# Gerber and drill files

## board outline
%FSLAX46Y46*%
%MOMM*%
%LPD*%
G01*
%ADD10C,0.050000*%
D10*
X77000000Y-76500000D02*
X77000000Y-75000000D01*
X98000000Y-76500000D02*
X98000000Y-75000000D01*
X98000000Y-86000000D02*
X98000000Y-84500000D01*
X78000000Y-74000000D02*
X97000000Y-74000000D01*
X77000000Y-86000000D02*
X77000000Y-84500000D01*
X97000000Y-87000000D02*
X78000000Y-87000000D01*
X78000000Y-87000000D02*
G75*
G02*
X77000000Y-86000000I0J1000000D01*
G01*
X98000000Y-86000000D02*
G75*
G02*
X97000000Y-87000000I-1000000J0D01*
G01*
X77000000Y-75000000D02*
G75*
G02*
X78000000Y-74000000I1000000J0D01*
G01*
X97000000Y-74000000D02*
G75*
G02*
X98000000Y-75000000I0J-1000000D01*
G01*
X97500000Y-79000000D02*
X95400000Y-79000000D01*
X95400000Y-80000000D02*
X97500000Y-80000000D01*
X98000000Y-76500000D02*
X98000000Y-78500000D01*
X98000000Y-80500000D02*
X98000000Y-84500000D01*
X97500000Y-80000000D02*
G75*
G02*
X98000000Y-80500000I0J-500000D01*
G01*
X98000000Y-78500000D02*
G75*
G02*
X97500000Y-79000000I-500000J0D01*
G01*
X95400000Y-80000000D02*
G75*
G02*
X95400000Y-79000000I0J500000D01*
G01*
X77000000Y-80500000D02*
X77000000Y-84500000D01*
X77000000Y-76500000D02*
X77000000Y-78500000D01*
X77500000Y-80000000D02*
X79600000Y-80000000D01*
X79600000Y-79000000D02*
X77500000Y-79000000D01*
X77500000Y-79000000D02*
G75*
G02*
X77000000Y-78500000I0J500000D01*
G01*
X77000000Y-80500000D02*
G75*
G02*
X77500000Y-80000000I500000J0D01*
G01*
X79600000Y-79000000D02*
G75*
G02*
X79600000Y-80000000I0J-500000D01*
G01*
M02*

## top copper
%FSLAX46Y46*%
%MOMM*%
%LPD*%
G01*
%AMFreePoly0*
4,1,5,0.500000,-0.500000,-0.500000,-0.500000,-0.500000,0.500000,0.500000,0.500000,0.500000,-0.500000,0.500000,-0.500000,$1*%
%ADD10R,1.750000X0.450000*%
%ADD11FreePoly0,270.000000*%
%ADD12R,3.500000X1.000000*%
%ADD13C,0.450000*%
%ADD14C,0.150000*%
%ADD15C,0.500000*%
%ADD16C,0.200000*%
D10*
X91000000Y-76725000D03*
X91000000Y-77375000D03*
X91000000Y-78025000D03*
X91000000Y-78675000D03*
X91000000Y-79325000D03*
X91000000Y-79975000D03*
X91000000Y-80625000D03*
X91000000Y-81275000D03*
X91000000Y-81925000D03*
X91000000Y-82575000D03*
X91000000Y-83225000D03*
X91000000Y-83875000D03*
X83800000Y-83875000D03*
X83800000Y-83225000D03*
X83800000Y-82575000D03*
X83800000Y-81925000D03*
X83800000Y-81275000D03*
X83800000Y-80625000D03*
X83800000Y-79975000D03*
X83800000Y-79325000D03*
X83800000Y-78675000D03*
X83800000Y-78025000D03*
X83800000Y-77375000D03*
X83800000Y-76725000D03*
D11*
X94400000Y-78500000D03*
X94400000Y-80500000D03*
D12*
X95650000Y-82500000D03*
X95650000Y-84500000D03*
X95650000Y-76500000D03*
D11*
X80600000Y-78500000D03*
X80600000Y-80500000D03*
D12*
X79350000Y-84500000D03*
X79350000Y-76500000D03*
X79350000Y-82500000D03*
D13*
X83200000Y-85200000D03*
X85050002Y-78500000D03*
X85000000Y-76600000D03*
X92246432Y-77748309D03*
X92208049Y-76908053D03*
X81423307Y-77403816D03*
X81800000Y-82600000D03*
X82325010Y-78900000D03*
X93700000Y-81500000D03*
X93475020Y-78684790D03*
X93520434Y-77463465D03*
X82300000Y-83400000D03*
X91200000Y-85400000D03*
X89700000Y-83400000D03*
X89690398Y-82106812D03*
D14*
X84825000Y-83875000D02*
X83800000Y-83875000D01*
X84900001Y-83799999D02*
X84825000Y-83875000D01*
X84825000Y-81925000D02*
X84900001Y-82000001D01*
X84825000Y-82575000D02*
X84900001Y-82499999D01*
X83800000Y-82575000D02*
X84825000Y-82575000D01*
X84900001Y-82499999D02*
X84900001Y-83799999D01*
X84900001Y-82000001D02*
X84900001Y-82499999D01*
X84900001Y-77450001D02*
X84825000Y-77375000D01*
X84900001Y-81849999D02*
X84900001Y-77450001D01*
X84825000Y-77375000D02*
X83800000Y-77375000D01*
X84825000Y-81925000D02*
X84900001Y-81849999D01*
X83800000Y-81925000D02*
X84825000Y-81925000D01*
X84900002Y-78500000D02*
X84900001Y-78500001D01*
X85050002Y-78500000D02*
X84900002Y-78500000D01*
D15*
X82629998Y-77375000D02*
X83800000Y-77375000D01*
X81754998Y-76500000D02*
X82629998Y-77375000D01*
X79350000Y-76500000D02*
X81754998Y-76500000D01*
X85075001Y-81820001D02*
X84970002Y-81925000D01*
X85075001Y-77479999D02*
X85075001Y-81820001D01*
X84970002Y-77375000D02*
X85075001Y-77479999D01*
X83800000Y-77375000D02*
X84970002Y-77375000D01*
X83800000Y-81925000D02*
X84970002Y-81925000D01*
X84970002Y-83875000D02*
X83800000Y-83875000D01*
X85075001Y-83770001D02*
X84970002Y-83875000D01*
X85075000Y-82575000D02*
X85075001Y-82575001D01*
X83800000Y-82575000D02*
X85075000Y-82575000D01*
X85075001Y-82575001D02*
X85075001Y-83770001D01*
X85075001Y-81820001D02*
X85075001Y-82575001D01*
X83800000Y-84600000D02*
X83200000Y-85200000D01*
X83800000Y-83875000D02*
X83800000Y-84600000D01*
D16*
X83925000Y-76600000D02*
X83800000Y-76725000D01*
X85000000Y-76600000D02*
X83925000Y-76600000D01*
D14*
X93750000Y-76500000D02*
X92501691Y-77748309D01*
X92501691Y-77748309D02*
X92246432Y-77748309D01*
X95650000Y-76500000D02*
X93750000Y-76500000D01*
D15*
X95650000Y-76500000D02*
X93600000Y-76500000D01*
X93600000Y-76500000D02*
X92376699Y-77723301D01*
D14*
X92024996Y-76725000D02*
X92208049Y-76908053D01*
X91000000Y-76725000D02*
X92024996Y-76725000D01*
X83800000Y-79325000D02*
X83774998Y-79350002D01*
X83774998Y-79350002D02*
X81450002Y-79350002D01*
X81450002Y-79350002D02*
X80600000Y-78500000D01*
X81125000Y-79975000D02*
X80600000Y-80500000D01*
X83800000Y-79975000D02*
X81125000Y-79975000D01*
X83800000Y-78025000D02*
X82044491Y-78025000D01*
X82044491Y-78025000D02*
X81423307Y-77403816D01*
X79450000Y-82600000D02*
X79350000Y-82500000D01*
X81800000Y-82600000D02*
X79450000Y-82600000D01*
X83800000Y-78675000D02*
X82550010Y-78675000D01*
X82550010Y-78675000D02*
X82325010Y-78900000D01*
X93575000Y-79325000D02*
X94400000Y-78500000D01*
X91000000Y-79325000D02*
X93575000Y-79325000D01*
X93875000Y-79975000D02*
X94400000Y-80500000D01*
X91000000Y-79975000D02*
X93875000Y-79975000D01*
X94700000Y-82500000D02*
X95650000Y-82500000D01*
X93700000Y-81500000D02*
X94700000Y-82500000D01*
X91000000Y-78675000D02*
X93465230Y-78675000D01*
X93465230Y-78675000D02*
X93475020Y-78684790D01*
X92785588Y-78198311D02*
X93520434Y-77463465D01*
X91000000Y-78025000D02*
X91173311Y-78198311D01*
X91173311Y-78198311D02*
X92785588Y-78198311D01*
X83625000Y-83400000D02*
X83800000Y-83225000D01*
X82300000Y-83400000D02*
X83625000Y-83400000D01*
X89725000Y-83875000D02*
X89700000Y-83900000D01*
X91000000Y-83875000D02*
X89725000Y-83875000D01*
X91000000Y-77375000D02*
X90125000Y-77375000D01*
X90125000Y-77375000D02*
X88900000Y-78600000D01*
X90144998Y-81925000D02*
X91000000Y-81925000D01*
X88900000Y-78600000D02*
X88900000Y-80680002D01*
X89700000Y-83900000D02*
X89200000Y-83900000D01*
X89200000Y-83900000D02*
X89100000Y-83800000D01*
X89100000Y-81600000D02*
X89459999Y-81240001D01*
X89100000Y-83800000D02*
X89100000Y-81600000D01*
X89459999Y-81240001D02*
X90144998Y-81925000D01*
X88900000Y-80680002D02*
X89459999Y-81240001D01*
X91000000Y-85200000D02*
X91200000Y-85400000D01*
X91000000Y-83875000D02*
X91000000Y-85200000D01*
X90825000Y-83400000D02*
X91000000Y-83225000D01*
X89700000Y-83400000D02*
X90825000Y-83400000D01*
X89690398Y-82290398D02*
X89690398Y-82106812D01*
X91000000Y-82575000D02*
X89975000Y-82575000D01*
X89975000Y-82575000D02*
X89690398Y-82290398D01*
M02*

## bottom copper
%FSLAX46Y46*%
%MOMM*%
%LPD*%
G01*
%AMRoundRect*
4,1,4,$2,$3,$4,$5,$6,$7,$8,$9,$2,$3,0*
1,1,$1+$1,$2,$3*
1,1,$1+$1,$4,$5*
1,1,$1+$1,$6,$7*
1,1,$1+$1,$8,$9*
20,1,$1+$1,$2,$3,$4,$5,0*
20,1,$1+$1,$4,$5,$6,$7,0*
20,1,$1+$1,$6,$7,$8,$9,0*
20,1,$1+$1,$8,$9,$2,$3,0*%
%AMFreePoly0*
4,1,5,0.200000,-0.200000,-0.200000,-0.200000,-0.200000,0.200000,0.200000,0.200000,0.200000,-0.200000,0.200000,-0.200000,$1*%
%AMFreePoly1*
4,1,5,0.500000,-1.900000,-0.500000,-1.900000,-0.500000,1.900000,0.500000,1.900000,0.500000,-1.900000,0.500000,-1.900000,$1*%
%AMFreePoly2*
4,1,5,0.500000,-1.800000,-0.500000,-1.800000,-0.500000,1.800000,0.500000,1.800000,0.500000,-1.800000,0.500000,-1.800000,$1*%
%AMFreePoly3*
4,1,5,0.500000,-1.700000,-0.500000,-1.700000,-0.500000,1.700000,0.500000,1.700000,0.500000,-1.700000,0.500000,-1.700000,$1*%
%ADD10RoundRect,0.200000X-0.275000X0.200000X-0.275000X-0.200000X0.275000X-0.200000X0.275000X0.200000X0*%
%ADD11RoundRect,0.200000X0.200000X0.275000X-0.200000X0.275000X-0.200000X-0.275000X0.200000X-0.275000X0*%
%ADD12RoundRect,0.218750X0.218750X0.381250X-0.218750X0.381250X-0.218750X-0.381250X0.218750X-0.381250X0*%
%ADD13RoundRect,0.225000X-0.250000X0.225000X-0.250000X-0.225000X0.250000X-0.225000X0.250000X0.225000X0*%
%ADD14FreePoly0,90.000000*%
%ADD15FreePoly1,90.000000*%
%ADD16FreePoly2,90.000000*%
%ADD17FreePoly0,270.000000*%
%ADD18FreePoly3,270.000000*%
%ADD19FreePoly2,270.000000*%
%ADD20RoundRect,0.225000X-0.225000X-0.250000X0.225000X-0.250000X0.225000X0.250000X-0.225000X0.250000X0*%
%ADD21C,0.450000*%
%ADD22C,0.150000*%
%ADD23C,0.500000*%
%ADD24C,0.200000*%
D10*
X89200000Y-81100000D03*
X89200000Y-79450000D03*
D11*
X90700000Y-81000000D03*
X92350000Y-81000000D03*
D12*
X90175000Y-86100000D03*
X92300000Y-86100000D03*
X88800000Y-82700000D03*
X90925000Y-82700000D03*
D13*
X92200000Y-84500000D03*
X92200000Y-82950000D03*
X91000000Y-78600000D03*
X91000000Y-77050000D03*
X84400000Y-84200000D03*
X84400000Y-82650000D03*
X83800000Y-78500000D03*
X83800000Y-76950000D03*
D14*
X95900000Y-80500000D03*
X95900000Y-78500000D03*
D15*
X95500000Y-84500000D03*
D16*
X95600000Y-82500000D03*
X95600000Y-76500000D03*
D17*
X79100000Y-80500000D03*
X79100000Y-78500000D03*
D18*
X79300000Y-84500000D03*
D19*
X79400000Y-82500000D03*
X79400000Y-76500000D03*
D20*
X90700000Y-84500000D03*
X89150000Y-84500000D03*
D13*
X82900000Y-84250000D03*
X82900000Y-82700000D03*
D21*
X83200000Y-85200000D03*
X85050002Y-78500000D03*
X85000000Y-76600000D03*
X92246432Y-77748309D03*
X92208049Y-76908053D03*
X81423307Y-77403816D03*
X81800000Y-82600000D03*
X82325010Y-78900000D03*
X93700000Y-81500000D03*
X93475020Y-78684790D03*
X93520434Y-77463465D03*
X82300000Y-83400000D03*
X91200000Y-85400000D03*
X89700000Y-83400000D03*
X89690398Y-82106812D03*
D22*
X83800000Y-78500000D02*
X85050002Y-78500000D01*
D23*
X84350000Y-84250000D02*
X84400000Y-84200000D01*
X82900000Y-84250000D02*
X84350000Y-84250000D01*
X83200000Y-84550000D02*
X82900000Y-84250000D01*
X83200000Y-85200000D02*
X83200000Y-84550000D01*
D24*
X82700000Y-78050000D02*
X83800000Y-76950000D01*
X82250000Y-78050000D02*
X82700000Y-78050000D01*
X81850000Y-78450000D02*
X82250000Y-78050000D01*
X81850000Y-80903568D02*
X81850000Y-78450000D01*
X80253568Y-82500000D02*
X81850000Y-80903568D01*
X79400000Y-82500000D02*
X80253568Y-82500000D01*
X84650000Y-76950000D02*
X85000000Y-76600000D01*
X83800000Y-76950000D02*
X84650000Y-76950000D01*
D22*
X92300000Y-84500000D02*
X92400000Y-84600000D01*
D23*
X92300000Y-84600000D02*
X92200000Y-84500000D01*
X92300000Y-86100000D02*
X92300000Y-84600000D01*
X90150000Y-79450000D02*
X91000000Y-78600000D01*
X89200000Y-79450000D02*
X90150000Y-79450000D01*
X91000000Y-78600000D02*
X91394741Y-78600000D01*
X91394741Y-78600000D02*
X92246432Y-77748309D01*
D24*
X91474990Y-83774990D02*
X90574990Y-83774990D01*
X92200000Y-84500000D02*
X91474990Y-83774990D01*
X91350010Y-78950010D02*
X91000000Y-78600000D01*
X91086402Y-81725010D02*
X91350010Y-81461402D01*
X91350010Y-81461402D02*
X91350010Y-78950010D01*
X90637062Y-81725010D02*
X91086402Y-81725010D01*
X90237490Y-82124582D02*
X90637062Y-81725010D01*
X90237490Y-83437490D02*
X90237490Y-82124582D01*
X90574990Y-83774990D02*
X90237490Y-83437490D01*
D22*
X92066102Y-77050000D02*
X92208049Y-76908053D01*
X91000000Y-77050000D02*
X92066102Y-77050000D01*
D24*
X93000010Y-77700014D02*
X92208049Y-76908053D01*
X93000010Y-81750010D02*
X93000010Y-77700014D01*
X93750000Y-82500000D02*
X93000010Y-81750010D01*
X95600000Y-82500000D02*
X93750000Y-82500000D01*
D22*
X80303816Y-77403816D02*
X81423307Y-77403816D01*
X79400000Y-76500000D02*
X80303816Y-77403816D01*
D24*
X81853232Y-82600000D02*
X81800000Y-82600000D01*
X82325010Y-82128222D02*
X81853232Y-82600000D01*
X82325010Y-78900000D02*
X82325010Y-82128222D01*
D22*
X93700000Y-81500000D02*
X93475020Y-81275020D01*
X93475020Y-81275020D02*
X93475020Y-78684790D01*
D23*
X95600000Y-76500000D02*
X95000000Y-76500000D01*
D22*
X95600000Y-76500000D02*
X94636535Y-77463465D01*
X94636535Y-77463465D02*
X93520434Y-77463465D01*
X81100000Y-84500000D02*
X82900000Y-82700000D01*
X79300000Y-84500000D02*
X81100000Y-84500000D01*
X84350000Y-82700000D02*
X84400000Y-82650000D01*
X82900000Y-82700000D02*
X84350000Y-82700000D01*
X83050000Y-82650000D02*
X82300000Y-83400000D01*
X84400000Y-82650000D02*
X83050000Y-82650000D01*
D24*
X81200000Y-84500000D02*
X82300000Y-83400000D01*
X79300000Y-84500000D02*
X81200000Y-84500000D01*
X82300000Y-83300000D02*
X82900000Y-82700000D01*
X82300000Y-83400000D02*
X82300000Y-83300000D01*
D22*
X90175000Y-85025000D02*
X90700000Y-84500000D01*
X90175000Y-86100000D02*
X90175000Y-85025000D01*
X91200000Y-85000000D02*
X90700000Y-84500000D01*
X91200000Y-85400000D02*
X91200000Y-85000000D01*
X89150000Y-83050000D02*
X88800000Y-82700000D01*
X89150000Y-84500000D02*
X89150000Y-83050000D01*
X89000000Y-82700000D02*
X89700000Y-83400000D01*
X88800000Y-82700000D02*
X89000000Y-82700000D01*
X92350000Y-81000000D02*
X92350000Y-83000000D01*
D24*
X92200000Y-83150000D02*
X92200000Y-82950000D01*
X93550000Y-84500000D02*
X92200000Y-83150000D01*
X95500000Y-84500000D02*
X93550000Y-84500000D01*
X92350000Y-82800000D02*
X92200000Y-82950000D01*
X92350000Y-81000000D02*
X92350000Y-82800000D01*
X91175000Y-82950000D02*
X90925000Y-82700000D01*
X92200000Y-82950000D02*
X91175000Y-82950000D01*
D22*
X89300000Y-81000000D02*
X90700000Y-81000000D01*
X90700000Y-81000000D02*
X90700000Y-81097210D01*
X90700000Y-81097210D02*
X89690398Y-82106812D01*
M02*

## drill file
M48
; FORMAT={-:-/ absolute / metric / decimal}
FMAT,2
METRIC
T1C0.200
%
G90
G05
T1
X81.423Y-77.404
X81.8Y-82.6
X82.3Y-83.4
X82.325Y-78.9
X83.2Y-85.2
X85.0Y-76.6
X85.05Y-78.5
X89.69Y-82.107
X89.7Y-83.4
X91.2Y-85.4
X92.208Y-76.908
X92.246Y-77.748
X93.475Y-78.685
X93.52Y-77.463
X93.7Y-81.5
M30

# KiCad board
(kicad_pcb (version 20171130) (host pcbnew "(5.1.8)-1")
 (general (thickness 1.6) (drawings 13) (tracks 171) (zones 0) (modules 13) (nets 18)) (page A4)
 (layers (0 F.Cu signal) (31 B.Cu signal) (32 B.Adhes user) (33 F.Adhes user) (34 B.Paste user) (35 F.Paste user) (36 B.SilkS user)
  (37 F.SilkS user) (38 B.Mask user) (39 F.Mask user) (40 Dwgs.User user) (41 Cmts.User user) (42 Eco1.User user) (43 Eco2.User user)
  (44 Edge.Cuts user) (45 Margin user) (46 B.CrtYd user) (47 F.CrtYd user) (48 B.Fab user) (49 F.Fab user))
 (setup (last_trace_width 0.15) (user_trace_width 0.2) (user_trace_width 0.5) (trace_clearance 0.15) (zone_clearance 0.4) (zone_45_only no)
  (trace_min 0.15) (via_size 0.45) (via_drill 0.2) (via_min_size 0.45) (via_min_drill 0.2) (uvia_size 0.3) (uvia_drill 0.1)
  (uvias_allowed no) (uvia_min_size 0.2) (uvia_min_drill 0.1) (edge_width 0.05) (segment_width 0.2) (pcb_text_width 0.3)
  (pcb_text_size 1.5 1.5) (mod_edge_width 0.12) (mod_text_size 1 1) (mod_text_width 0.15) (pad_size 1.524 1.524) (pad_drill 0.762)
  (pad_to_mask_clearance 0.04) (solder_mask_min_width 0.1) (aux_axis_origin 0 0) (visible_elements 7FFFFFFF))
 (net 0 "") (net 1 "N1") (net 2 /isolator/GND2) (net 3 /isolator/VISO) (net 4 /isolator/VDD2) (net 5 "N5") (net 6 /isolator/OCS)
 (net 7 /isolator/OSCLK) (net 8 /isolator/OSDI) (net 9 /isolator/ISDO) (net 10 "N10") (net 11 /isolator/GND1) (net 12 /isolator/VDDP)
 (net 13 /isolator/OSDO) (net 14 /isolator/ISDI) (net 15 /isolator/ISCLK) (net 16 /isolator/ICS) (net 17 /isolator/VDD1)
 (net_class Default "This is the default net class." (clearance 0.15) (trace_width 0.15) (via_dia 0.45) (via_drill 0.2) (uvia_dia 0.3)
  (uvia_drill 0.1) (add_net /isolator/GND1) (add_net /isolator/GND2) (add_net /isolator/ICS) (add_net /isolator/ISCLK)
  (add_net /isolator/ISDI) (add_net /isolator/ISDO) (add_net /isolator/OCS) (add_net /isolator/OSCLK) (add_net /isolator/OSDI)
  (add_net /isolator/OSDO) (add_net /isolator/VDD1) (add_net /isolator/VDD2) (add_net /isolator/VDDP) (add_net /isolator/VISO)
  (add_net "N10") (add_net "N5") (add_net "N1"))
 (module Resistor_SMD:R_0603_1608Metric (layer B.Cu) (at 89.2 80.275 270)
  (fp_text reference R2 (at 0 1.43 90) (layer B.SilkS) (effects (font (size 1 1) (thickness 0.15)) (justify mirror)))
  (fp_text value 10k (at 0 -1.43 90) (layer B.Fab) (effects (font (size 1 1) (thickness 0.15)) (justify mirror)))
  (pad 2 smd roundrect (at 0.825 0 270) (size 0.8 0.95) (layers B.Cu B.Paste B.Mask) (roundrect_rratio 0.25) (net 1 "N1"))
  (pad 1 smd roundrect (at -0.825 0 270) (size 0.8 0.95) (layers B.Cu B.Paste B.Mask) (roundrect_rratio 0.25) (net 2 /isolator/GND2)))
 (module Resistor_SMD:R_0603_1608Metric (layer B.Cu) (at 91.525 81 180)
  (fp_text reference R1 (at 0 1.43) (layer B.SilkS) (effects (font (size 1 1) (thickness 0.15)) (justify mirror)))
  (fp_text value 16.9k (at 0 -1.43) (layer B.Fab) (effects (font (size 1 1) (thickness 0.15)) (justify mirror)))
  (pad 2 smd roundrect (at 0.825 0 180) (size 0.8 0.95) (layers B.Cu B.Paste B.Mask) (roundrect_rratio 0.25) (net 1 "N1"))
  (pad 1 smd roundrect (at -0.825 0 180) (size 0.8 0.95) (layers B.Cu B.Paste B.Mask) (roundrect_rratio 0.25) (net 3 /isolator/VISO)))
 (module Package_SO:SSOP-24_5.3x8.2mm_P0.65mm (layer F.Cu) (at 87.4 80.3)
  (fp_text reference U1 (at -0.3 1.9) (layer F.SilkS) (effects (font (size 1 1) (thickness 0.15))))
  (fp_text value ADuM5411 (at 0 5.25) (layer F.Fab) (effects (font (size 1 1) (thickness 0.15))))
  (pad 24 smd rect (at 3.6 -3.575) (size 1.75 0.45) (layers F.Cu F.Paste F.Mask) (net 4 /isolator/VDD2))
  (pad 23 smd rect (at 3.6 -2.925) (size 1.75 0.45) (layers F.Cu F.Paste F.Mask) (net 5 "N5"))
  (pad 22 smd rect (at 3.6 -2.275) (size 1.75 0.45) (layers F.Cu F.Paste F.Mask) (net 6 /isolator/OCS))
  (pad 21 smd rect (at 3.6 -1.625) (size 1.75 0.45) (layers F.Cu F.Paste F.Mask) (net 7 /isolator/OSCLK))
  (pad 20 smd rect (at 3.6 -0.975) (size 1.75 0.45) (layers F.Cu F.Paste F.Mask) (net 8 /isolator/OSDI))
  (pad 19 smd rect (at 3.6 -0.325) (size 1.75 0.45) (layers F.Cu F.Paste F.Mask) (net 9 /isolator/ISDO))
  (pad 18 smd rect (at 3.6 0.325) (size 1.75 0.45) (layers F.Cu F.Paste F.Mask))
  (pad 17 smd rect (at 3.6 0.975) (size 1.75 0.45) (layers F.Cu F.Paste F.Mask))
  (pad 16 smd rect (at 3.6 1.625) (size 1.75 0.45) (layers F.Cu F.Paste F.Mask) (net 5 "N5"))
  (pad 15 smd rect (at 3.6 2.275) (size 1.75 0.45) (layers F.Cu F.Paste F.Mask) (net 1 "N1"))
  (pad 14 smd rect (at 3.6 2.925) (size 1.75 0.45) (layers F.Cu F.Paste F.Mask) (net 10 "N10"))
  (pad 13 smd rect (at 3.6 3.575) (size 1.75 0.45) (layers F.Cu F.Paste F.Mask) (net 5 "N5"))
  (pad 12 smd rect (at -3.6 3.575) (size 1.75 0.45) (layers F.Cu F.Paste F.Mask) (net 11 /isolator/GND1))
  (pad 11 smd rect (at -3.6 2.925) (size 1.75 0.45) (layers F.Cu F.Paste F.Mask) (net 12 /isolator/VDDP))
  (pad 10 smd rect (at -3.6 2.275) (size 1.75 0.45) (layers F.Cu F.Paste F.Mask) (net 11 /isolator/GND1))
  (pad 9 smd rect (at -3.6 1.625) (size 1.75 0.45) (layers F.Cu F.Paste F.Mask) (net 11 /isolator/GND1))
  (pad 8 smd rect (at -3.6 0.975) (size 1.75 0.45) (layers F.Cu F.Paste F.Mask))
  (pad 7 smd rect (at -3.6 0.325) (size 1.75 0.45) (layers F.Cu F.Paste F.Mask))
  (pad 6 smd rect (at -3.6 -0.325) (size 1.75 0.45) (layers F.Cu F.Paste F.Mask) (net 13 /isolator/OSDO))
  (pad 5 smd rect (at -3.6 -0.975) (size 1.75 0.45) (layers F.Cu F.Paste F.Mask) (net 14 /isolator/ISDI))
  (pad 4 smd rect (at -3.6 -1.625) (size 1.75 0.45) (layers F.Cu F.Paste F.Mask) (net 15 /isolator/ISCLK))
  (pad 3 smd rect (at -3.6 -2.275) (size 1.75 0.45) (layers F.Cu F.Paste F.Mask) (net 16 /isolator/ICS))
  (pad 2 smd rect (at -3.6 -2.925) (size 1.75 0.45) (layers F.Cu F.Paste F.Mask) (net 11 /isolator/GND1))
  (pad 1 smd rect (at -3.6 -3.575) (size 1.75 0.45) (layers F.Cu F.Paste F.Mask) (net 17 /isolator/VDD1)))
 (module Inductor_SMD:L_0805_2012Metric (layer B.Cu) (at 91.2375 86.1 180)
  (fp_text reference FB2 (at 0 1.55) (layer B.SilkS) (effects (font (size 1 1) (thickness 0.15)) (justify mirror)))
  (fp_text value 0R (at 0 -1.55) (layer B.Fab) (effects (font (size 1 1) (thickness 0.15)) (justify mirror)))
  (pad 2 smd roundrect (at 1.0625 0 180) (size 0.875 1.2) (layers B.Cu B.Paste B.Mask) (roundrect_rratio 0.25) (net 5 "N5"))
  (pad 1 smd roundrect (at -1.0625 0 180) (size 0.875 1.2) (layers B.Cu B.Paste B.Mask) (roundrect_rratio 0.25) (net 2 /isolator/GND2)))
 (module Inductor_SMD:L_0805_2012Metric (layer B.Cu) (at 89.8625 82.7 180)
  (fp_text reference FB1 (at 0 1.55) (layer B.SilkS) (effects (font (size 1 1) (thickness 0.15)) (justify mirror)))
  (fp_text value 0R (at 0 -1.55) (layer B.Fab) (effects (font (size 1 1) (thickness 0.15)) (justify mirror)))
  (pad 2 smd roundrect (at 1.0625 0 180) (size 0.875 1.2) (layers B.Cu B.Paste B.Mask) (roundrect_rratio 0.25) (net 10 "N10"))
  (pad 1 smd roundrect (at -1.0625 0 180) (size 0.875 1.2) (layers B.Cu B.Paste B.Mask) (roundrect_rratio 0.25) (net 3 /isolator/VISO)))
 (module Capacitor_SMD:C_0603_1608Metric (layer B.Cu) (at 92.2 83.725 270)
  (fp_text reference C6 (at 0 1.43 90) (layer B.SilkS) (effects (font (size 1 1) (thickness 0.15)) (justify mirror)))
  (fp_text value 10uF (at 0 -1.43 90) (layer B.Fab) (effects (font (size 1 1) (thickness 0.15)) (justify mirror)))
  (pad 2 smd roundrect (at 0.775 0 270) (size 0.9 0.95) (layers B.Cu B.Paste B.Mask) (roundrect_rratio 0.25) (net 2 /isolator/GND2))
  (pad 1 smd roundrect (at -0.775 0 270) (size 0.9 0.95) (layers B.Cu B.Paste B.Mask) (roundrect_rratio 0.25) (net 3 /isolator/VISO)))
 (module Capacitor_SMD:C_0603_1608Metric (layer B.Cu) (at 91 77.825 270)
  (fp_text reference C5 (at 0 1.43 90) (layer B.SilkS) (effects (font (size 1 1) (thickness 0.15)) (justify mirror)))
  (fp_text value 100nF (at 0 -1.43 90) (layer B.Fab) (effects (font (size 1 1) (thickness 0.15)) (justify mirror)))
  (pad 2 smd roundrect (at 0.775 0 270) (size 0.9 0.95) (layers B.Cu B.Paste B.Mask) (roundrect_rratio 0.25) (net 2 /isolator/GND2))
  (pad 1 smd roundrect (at -0.775 0 270) (size 0.9 0.95) (layers B.Cu B.Paste B.Mask) (roundrect_rratio 0.25) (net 4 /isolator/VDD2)))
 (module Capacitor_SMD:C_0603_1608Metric (layer B.Cu) (at 84.4 83.425 270)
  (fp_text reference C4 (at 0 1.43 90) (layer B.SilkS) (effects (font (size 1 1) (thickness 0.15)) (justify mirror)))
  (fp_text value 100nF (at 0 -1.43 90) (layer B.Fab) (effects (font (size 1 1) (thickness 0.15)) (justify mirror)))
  (pad 2 smd roundrect (at 0.775 0 270) (size 0.9 0.95) (layers B.Cu B.Paste B.Mask) (roundrect_rratio 0.25) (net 11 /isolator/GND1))
  (pad 1 smd roundrect (at -0.775 0 270) (size 0.9 0.95) (layers B.Cu B.Paste B.Mask) (roundrect_rratio 0.25) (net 12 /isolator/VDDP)))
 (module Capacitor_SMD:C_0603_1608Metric (layer B.Cu) (at 83.8 77.725 270)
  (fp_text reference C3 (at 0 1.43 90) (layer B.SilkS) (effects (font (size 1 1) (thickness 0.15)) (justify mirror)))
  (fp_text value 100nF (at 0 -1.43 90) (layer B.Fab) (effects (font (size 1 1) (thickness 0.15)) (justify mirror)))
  (pad 2 smd roundrect (at 0.775 0 270) (size 0.9 0.95) (layers B.Cu B.Paste B.Mask) (roundrect_rratio 0.25) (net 11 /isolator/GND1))
  (pad 1 smd roundrect (at -0.775 0 270) (size 0.9 0.95) (layers B.Cu B.Paste B.Mask) (roundrect_rratio 0.25) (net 17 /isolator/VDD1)))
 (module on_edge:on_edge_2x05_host (layer F.Cu) (at 98 80.5 270)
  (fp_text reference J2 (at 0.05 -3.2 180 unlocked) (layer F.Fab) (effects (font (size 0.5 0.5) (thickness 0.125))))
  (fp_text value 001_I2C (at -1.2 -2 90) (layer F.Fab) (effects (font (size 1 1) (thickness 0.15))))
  (fp_line (start -1.5 0.5) (end -1.5 2.6) (layer Edge.Cuts) (width 0.05))
  (fp_line (start -0.5 2.6) (end -0.5 0.5) (layer Edge.Cuts) (width 0.05))
  (fp_line (start -4 0) (end -2 0) (layer Edge.Cuts) (width 0.05))
  (fp_line (start 0 0) (end 4 0) (layer Edge.Cuts) (width 0.05))
  (fp_arc (start 0 0.5) (end 0 0) (angle -90) (layer Edge.Cuts) (width 0.05))
  (fp_arc (start -2 0.5) (end -1.5 0.5) (angle -90) (layer Edge.Cuts) (width 0.05))
  (fp_arc (start -1 2.6) (end -1.5 2.6) (angle -180) (layer Edge.Cuts) (width 0.05))
  (pad 2 smd custom (at -2 3.6 270) (size 1 1) (layers F.Cu F.Mask) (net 8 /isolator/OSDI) (zone_connect 0)
   (options (clearance outline) (anchor rect)) (primitives))
  (pad 3 smd custom (at 0 3.6 270) (size 1 1) (layers F.Cu F.Mask) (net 9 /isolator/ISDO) (zone_connect 0)
   (options (clearance outline) (anchor rect)) (primitives))
  (pad 8 smd custom (at 0 2.1 90) (size 0.4 0.4) (layers B.Cu B.Mask) (zone_connect 0) (options (clearance outline) (anchor rect))
   (primitives))
  (pad 7 smd custom (at -2 2.1 90) (size 0.4 0.4) (layers B.Cu B.Mask) (zone_connect 0) (options (clearance outline) (anchor rect))
   (primitives))
  (pad 4 smd rect (at 2 2.35 270) (size 1 3.5) (layers F.Cu F.Mask) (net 7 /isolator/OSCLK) (zone_connect 0))
  (pad 10 smd custom (at 4 2.5 90) (size 1 3.8) (layers B.Cu B.Mask) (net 3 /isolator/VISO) (zone_connect 0)
   (options (clearance outline) (anchor rect)) (primitives))
  (pad 9 smd custom (at 2 2.4 90) (size 1 3.6) (layers B.Cu B.Mask) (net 4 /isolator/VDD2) (zone_connect 0)
   (options (clearance outline) (anchor rect)) (primitives))
  (pad 6 smd custom (at -4 2.4 90) (size 1 3.6) (layers B.Cu B.Mask) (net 6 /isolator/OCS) (zone_connect 0)
   (options (clearance outline) (anchor rect)) (primitives))
  (pad 5 smd rect (at 4 2.35 270) (size 1 3.5) (layers F.Cu F.Mask) (zone_connect 0))
  (pad 1 smd rect (at -4 2.35 270) (size 1 3.5) (layers F.Cu F.Mask) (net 2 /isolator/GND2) (zone_connect 0)))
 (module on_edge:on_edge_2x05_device (layer F.Cu) (at 77 80.5 270)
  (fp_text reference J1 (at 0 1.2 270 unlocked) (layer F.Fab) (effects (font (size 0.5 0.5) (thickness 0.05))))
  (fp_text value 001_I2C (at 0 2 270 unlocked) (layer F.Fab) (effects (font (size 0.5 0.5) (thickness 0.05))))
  (fp_line (start 0 0) (end 4 0) (layer Edge.Cuts) (width 0.05))
  (fp_line (start -4 0) (end -2 0) (layer Edge.Cuts) (width 0.05))
  (fp_line (start -0.5 -0.5) (end -0.5 -2.6) (layer Edge.Cuts) (width 0.05))
  (fp_line (start -1.5 -2.6) (end -1.5 -0.5) (layer Edge.Cuts) (width 0.05))
  (fp_arc (start -2 -0.5) (end -2 0) (angle -90) (layer Edge.Cuts) (width 0.05))
  (fp_arc (start 0 -0.5) (end -0.5 -0.5) (angle -90) (layer Edge.Cuts) (width 0.05))
  (fp_arc (start -1 -2.6) (end -0.5 -2.6) (angle -180) (layer Edge.Cuts) (width 0.05))
  (pad 2 smd custom (at -2 -3.6 270) (size 1 1) (layers F.Cu F.Mask) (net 14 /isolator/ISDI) (zone_connect 0)
   (options (clearance outline) (anchor rect)) (primitives))
  (pad 3 smd custom (at 0 -3.6 270) (size 1 1) (layers F.Cu F.Mask) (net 13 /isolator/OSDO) (zone_connect 0)
   (options (clearance outline) (anchor rect)) (primitives))
  (pad 8 smd custom (at 0 -2.1 270) (size 0.4 0.4) (layers B.Cu B.Mask) (zone_connect 0) (options (clearance outline) (anchor rect))
   (primitives))
  (pad 7 smd custom (at -2 -2.1 270) (size 0.4 0.4) (layers B.Cu B.Mask) (zone_connect 0) (options (clearance outline) (anchor rect))
   (primitives))
  (pad 10 smd custom (at 4 -2.3 270) (size 1 3.4) (layers B.Cu B.Mask) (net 12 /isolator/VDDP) (zone_connect 0)
   (options (clearance outline) (anchor rect)) (primitives))
  (pad 9 smd custom (at 2 -2.4 270) (size 1 3.6) (layers B.Cu B.Mask) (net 17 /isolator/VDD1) (zone_connect 0)
   (options (clearance outline) (anchor rect)) (primitives))
  (pad 6 smd custom (at -4 -2.4 270) (size 1 3.6) (layers B.Cu B.Mask) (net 16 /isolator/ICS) (zone_connect 0)
   (options (clearance outline) (anchor rect)) (primitives))
  (pad 5 smd rect (at 4 -2.35 90) (size 1 3.5) (layers F.Cu F.Mask) (zone_connect 0))
  (pad 1 smd rect (at -4 -2.35 90) (size 1 3.5) (layers F.Cu F.Mask) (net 11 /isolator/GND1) (zone_connect 0))
  (pad 4 smd rect (at 2 -2.35 90) (size 1 3.5) (layers F.Cu F.Mask) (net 15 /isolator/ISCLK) (zone_connect 0)))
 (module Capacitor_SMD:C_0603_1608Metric (layer B.Cu) (at 89.925 84.5)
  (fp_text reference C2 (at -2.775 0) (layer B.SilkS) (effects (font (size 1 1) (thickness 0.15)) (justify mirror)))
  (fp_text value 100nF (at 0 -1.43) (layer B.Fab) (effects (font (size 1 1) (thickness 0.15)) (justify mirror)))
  (pad 2 smd roundrect (at 0.775 0) (size 0.9 0.95) (layers B.Cu B.Paste B.Mask) (roundrect_rratio 0.25) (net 5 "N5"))
  (pad 1 smd roundrect (at -0.775 0) (size 0.9 0.95) (layers B.Cu B.Paste B.Mask) (roundrect_rratio 0.25) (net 10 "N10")))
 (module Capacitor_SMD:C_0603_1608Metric (layer B.Cu) (at 82.9 83.475 270)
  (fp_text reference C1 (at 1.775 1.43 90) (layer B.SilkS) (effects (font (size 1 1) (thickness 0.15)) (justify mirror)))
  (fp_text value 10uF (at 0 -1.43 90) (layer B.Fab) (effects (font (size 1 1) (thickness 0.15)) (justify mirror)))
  (pad 2 smd roundrect (at 0.775 0 270) (size 0.9 0.95) (layers B.Cu B.Paste B.Mask) (roundrect_rratio 0.25) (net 11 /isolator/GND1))
  (pad 1 smd roundrect (at -0.775 0 270) (size 0.9 0.95) (layers B.Cu B.Paste B.Mask) (roundrect_rratio 0.25) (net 12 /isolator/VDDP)))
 (gr_line (start 77 76.5) (end 77 75) (layer Edge.Cuts) (width 0.05))
 (gr_line (start 98 76.5) (end 98 75) (layer Edge.Cuts) (width 0.05))
 (gr_line (start 98 86) (end 98 84.5) (layer Edge.Cuts) (width 0.05))
 (gr_line (start 78 74) (end 97 74) (layer Edge.Cuts) (width 0.05))
 (gr_line (start 77 86) (end 77 84.5) (layer Edge.Cuts) (width 0.05))
 (gr_line (start 97 87) (end 78 87) (layer Edge.Cuts) (width 0.05))
 (gr_arc (start 78 86) (end 77 86) (angle -90) (layer Edge.Cuts) (width 0.05))
 (gr_arc (start 97 86) (end 97 87) (angle -90) (layer Edge.Cuts) (width 0.05))
 (gr_arc (start 78 75) (end 78 74) (angle -90) (layer Edge.Cuts) (width 0.05))
 (gr_arc (start 97 75) (end 98 75) (angle -90) (layer Edge.Cuts) (width 0.05))
 (via (at 83.2 85.2) (size 0.45) (drill 0.2) (layers F.Cu B.Cu) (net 11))
 (segment (start 84.825 83.875) (end 83.8 83.875) (width 0.15) (layer F.Cu) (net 11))
 (segment (start 84.900001 83.799999) (end 84.825 83.875) (width 0.15) (layer F.Cu) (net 11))
 (segment (start 84.825 81.925) (end 84.900001 82.000001) (width 0.15) (layer F.Cu) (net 11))
 (segment (start 84.825 82.575) (end 84.900001 82.499999) (width 0.15) (layer F.Cu) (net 11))
 (segment (start 83.8 82.575) (end 84.825 82.575) (width 0.15) (layer F.Cu) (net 11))
 (segment (start 84.900001 82.499999) (end 84.900001 83.799999) (width 0.15) (layer F.Cu) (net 11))
 (segment (start 84.900001 82.000001) (end 84.900001 82.499999) (width 0.15) (layer F.Cu) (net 11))
 (segment (start 84.900001 77.450001) (end 84.825 77.375) (width 0.15) (layer F.Cu) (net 11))
 (segment (start 84.900001 81.849999) (end 84.900001 77.450001) (width 0.15) (layer F.Cu) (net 11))
 (segment (start 84.825 77.375) (end 83.8 77.375) (width 0.15) (layer F.Cu) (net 11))
 (segment (start 84.825 81.925) (end 84.900001 81.849999) (width 0.15) (layer F.Cu) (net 11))
 (segment (start 83.8 81.925) (end 84.825 81.925) (width 0.15) (layer F.Cu) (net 11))
 (via (at 85.050002 78.5) (size 0.45) (drill 0.2) (layers F.Cu B.Cu) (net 11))
 (segment (start 83.8 78.5) (end 85.050002 78.5) (width 0.15) (layer B.Cu) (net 11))
 (segment (start 84.900002 78.5) (end 84.900001 78.500001) (width 0.15) (layer F.Cu) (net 11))
 (segment (start 85.050002 78.5) (end 84.900002 78.5) (width 0.15) (layer F.Cu) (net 11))
 (segment (start 82.629998 77.375) (end 83.8 77.375) (width 0.5) (layer F.Cu) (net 11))
 (segment (start 81.754998 76.5) (end 82.629998 77.375) (width 0.5) (layer F.Cu) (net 11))
 (segment (start 79.35 76.5) (end 81.754998 76.5) (width 0.5) (layer F.Cu) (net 11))
 (segment (start 85.075001 81.820001) (end 84.970002 81.925) (width 0.5) (layer F.Cu) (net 11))
 (segment (start 85.075001 77.479999) (end 85.075001 81.820001) (width 0.5) (layer F.Cu) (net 11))
 (segment (start 84.970002 77.375) (end 85.075001 77.479999) (width 0.5) (layer F.Cu) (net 11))
 (segment (start 83.8 77.375) (end 84.970002 77.375) (width 0.5) (layer F.Cu) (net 11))
 (segment (start 83.8 81.925) (end 84.970002 81.925) (width 0.5) (layer F.Cu) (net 11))
 (segment (start 84.970002 83.875) (end 83.8 83.875) (width 0.5) (layer F.Cu) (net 11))
 (segment (start 85.075001 83.770001) (end 84.970002 83.875) (width 0.5) (layer F.Cu) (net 11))
 (segment (start 85.075 82.575) (end 85.075001 82.575001) (width 0.5) (layer F.Cu) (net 11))
 (segment (start 83.8 82.575) (end 85.075 82.575) (width 0.5) (layer F.Cu) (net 11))
 (segment (start 85.075001 82.575001) (end 85.075001 83.770001) (width 0.5) (layer F.Cu) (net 11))
 (segment (start 85.075001 81.820001) (end 85.075001 82.575001) (width 0.5) (layer F.Cu) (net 11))
 (segment (start 83.8 84.6) (end 83.2 85.2) (width 0.5) (layer F.Cu) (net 11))
 (segment (start 83.8 83.875) (end 83.8 84.6) (width 0.5) (layer F.Cu) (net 11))
 (segment (start 84.35 84.25) (end 84.4 84.2) (width 0.5) (layer B.Cu) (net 11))
 (segment (start 82.9 84.25) (end 84.35 84.25) (width 0.5) (layer B.Cu) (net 11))
 (segment (start 83.2 84.55) (end 82.9 84.25) (width 0.5) (layer B.Cu) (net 11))
 (segment (start 83.2 85.2) (end 83.2 84.55) (width 0.5) (layer B.Cu) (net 11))
 (via (at 85 76.6) (size 0.45) (drill 0.2) (layers F.Cu B.Cu) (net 17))
 (segment (start 82.7 78.05) (end 83.8 76.95) (width 0.2) (layer B.Cu) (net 17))
 (segment (start 82.25 78.05) (end 82.7 78.05) (width 0.2) (layer B.Cu) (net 17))
 (segment (start 81.85 78.45) (end 82.25 78.05) (width 0.2) (layer B.Cu) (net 17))
 (segment (start 81.85 80.903568) (end 81.85 78.45) (width 0.2) (layer B.Cu) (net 17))
 (segment (start 80.253568 82.5) (end 81.85 80.903568) (width 0.2) (layer B.Cu) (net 17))
 (segment (start 79.4 82.5) (end 80.253568 82.5) (width 0.2) (layer B.Cu) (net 17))
 (segment (start 84.65 76.95) (end 85 76.6) (width 0.2) (layer B.Cu) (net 17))
 (segment (start 83.8 76.95) (end 84.65 76.95) (width 0.2) (layer B.Cu) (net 17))
 (segment (start 83.925 76.6) (end 83.8 76.725) (width 0.2) (layer F.Cu) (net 17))
 (segment (start 85 76.6) (end 83.925 76.6) (width 0.2) (layer F.Cu) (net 17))
 (segment (start 92.3 84.5) (end 92.4 84.6) (width 0.15) (layer B.Cu) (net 2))
 (via (at 92.246432 77.748309) (size 0.45) (drill 0.2) (layers F.Cu B.Cu) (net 2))
 (segment (start 93.75 76.5) (end 92.501691 77.748309) (width 0.15) (layer F.Cu) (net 2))
 (segment (start 92.501691 77.748309) (end 92.246432 77.748309) (width 0.15) (layer F.Cu) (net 2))
 (segment (start 95.65 76.5) (end 93.75 76.5) (width 0.15) (layer F.Cu) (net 2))
 (segment (start 92.3 84.6) (end 92.2 84.5) (width 0.5) (layer B.Cu) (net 2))
 (segment (start 92.3 86.1) (end 92.3 84.6) (width 0.5) (layer B.Cu) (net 2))
 (segment (start 90.15 79.45) (end 91 78.6) (width 0.5) (layer B.Cu) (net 2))
 (segment (start 89.2 79.45) (end 90.15 79.45) (width 0.5) (layer B.Cu) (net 2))
 (segment (start 91 78.6) (end 91.394741 78.6) (width 0.5) (layer B.Cu) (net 2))
 (segment (start 91.394741 78.6) (end 92.246432 77.748309) (width 0.5) (layer B.Cu) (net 2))
 (segment (start 95.65 76.5) (end 93.6 76.5) (width 0.5) (layer F.Cu) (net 2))
 (segment (start 93.6 76.5) (end 92.376699 77.723301) (width 0.5) (layer F.Cu) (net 2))
 (segment (start 91.47499 83.77499) (end 90.57499 83.77499) (width 0.2) (layer B.Cu) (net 2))
 (segment (start 92.2 84.5) (end 91.47499 83.77499) (width 0.2) (layer B.Cu) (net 2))
 (segment (start 91.35001 78.95001) (end 91 78.6) (width 0.2) (layer B.Cu) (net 2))
 (segment (start 91.086402 81.72501) (end 91.35001 81.461402) (width 0.2) (layer B.Cu) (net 2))
 (segment (start 91.35001 81.461402) (end 91.35001 78.95001) (width 0.2) (layer B.Cu) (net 2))
 (segment (start 90.637062 81.72501) (end 91.086402 81.72501) (width 0.2) (layer B.Cu) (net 2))
 (segment (start 90.23749 82.124582) (end 90.637062 81.72501) (width 0.2) (layer B.Cu) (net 2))
 (segment (start 90.23749 83.43749) (end 90.23749 82.124582) (width 0.2) (layer B.Cu) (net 2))
 (segment (start 90.57499 83.77499) (end 90.23749 83.43749) (width 0.2) (layer B.Cu) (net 2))
 (segment (start 92.066102 77.05) (end 92.208049 76.908053) (width 0.15) (layer B.Cu) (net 4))
 (segment (start 91 77.05) (end 92.066102 77.05) (width 0.15) (layer B.Cu) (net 4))
 (segment (start 92.024996 76.725) (end 92.208049 76.908053) (width 0.15) (layer F.Cu) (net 4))
 (segment (start 91 76.725) (end 92.024996 76.725) (width 0.15) (layer F.Cu) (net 4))
 (via (at 92.208049 76.908053) (size 0.45) (drill 0.2) (layers F.Cu B.Cu) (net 4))
 (segment (start 93.00001 77.700014) (end 92.208049 76.908053) (width 0.2) (layer B.Cu) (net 4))
 (segment (start 93.00001 81.75001) (end 93.00001 77.700014) (width 0.2) (layer B.Cu) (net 4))
 (segment (start 93.75 82.5) (end 93.00001 81.75001) (width 0.2) (layer B.Cu) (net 4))
 (segment (start 95.6 82.5) (end 93.75 82.5) (width 0.2) (layer B.Cu) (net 4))
 (segment (start 83.8 79.325) (end 83.774998 79.350002) (width 0.15) (layer F.Cu) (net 14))
 (segment (start 83.774998 79.350002) (end 81.450002 79.350002) (width 0.15) (layer F.Cu) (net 14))
 (segment (start 81.450002 79.350002) (end 80.6 78.5) (width 0.15) (layer F.Cu) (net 14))
 (segment (start 81.125 79.975) (end 80.6 80.5) (width 0.15) (layer F.Cu) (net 13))
 (segment (start 83.8 79.975) (end 81.125 79.975) (width 0.15) (layer F.Cu) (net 13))
 (via (at 81.423307 77.403816) (size 0.45) (drill 0.2) (layers F.Cu B.Cu) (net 16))
 (segment (start 83.8 78.025) (end 82.044491 78.025) (width 0.15) (layer F.Cu) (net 16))
 (segment (start 80.303816 77.403816) (end 81.423307 77.403816) (width 0.15) (layer B.Cu) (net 16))
 (segment (start 82.044491 78.025) (end 81.423307 77.403816) (width 0.15) (layer F.Cu) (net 16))
 (segment (start 79.4 76.5) (end 80.303816 77.403816) (width 0.15) (layer B.Cu) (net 16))
 (via (at 81.8 82.6) (size 0.45) (drill 0.2) (layers F.Cu B.Cu) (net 15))
 (segment (start 79.45 82.6) (end 79.35 82.5) (width 0.15) (layer F.Cu) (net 15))
 (segment (start 81.8 82.6) (end 79.45 82.6) (width 0.15) (layer F.Cu) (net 15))
 (via (at 82.32501 78.9) (size 0.45) (drill 0.2) (layers F.Cu B.Cu) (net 15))
 (segment (start 83.8 78.675) (end 82.55001 78.675) (width 0.15) (layer F.Cu) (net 15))
 (segment (start 82.55001 78.675) (end 82.32501 78.9) (width 0.15) (layer F.Cu) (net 15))
 (segment (start 81.853232 82.6) (end 81.8 82.6) (width 0.2) (layer B.Cu) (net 15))
 (segment (start 82.32501 82.128222) (end 81.853232 82.6) (width 0.2) (layer B.Cu) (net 15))
 (segment (start 82.32501 78.9) (end 82.32501 82.128222) (width 0.2) (layer B.Cu) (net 15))
 (segment (start 93.575 79.325) (end 94.4 78.5) (width 0.15) (layer F.Cu) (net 8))
 (segment (start 91 79.325) (end 93.575 79.325) (width 0.15) (layer F.Cu) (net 8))
 (segment (start 93.875 79.975) (end 94.4 80.5) (width 0.15) (layer F.Cu) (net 9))
 (segment (start 91 79.975) (end 93.875 79.975) (width 0.15) (layer F.Cu) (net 9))
 (via (at 93.7 81.5) (size 0.45) (drill 0.2) (layers F.Cu B.Cu) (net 7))
 (segment (start 94.7 82.5) (end 95.65 82.5) (width 0.15) (layer F.Cu) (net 7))
 (segment (start 93.7 81.5) (end 94.7 82.5) (width 0.15) (layer F.Cu) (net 7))
 (via (at 93.47502 78.68479) (size 0.45) (drill 0.2) (layers F.Cu B.Cu) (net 7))
 (segment (start 91 78.675) (end 93.46523 78.675) (width 0.15) (layer F.Cu) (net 7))
 (segment (start 93.46523 78.675) (end 93.47502 78.68479) (width 0.15) (layer F.Cu) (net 7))
 (segment (start 93.7 81.5) (end 93.47502 81.27502) (width 0.15) (layer B.Cu) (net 7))
 (segment (start 93.47502 81.27502) (end 93.47502 78.68479) (width 0.15) (layer B.Cu) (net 7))
 (segment (start 95.6 76.5) (end 95 76.5) (width 0.5) (layer B.Cu) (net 6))
 (segment (start 95.6 76.5) (end 94.636535 77.463465) (width 0.15) (layer B.Cu) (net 6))
 (segment (start 92.785588 78.198311) (end 93.520434 77.463465) (width 0.15) (layer F.Cu) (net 6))
 (segment (start 94.636535 77.463465) (end 93.520434 77.463465) (width 0.15) (layer B.Cu) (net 6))
 (segment (start 91 78.025) (end 91.173311 78.198311) (width 0.15) (layer F.Cu) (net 6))
 (via (at 93.520434 77.463465) (size 0.45) (drill 0.2) (layers F.Cu B.Cu) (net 6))
 (segment (start 91.173311 78.198311) (end 92.785588 78.198311) (width 0.15) (layer F.Cu) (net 6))
 (segment (start 81.1 84.5) (end 82.9 82.7) (width 0.15) (layer B.Cu) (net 12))
 (segment (start 79.3 84.5) (end 81.1 84.5) (width 0.15) (layer B.Cu) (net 12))
 (segment (start 84.35 82.7) (end 84.4 82.65) (width 0.15) (layer B.Cu) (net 12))
 (segment (start 82.9 82.7) (end 84.35 82.7) (width 0.15) (layer B.Cu) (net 12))
 (via (at 82.3 83.4) (size 0.45) (drill 0.2) (layers F.Cu B.Cu) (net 12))
 (segment (start 83.05 82.65) (end 82.3 83.4) (width 0.15) (layer B.Cu) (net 12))
 (segment (start 84.4 82.65) (end 83.05 82.65) (width 0.15) (layer B.Cu) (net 12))
 (segment (start 83.625 83.4) (end 83.8 83.225) (width 0.15) (layer F.Cu) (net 12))
 (segment (start 82.3 83.4) (end 83.625 83.4) (width 0.15) (layer F.Cu) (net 12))
 (segment (start 81.2 84.5) (end 82.3 83.4) (width 0.2) (layer B.Cu) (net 12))
 (segment (start 79.3 84.5) (end 81.2 84.5) (width 0.2) (layer B.Cu) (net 12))
 (segment (start 82.3 83.3) (end 82.9 82.7) (width 0.2) (layer B.Cu) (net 12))
 (segment (start 82.3 83.4) (end 82.3 83.3) (width 0.2) (layer B.Cu) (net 12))
 (segment (start 89.725 83.875) (end 89.7 83.9) (width 0.15) (layer F.Cu) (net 5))
 (segment (start 91 83.875) (end 89.725 83.875) (width 0.15) (layer F.Cu) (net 5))
 (segment (start 91 77.375) (end 90.125 77.375) (width 0.15) (layer F.Cu) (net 5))
 (segment (start 90.125 77.375) (end 88.9 78.6) (width 0.15) (layer F.Cu) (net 5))
 (segment (start 90.144998 81.925) (end 91 81.925) (width 0.15) (layer F.Cu) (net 5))
 (segment (start 88.9 78.6) (end 88.9 80.680002) (width 0.15) (layer F.Cu) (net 5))
 (segment (start 89.7 83.9) (end 89.2 83.9) (width 0.15) (layer F.Cu) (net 5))
 (segment (start 89.2 83.9) (end 89.1 83.8) (width 0.15) (layer F.Cu) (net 5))
 (segment (start 89.1 81.6) (end 89.459999 81.240001) (width 0.15) (layer F.Cu) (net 5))
 (segment (start 89.1 83.8) (end 89.1 81.6) (width 0.15) (layer F.Cu) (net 5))
 (segment (start 89.459999 81.240001) (end 90.144998 81.925) (width 0.15) (layer F.Cu) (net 5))
 (segment (start 88.9 80.680002) (end 89.459999 81.240001) (width 0.15) (layer F.Cu) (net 5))
 (segment (start 90.175 85.025) (end 90.7 84.5) (width 0.15) (layer B.Cu) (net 5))
 (segment (start 90.175 86.1) (end 90.175 85.025) (width 0.15) (layer B.Cu) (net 5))
 (via (at 91.2 85.4) (size 0.45) (drill 0.2) (layers F.Cu B.Cu) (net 5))
 (segment (start 91 85.2) (end 91.2 85.4) (width 0.15) (layer F.Cu) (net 5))
 (segment (start 91 83.875) (end 91 85.2) (width 0.15) (layer F.Cu) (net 5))
 (segment (start 91.2 85) (end 90.7 84.5) (width 0.15) (layer B.Cu) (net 5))
 (segment (start 91.2 85.4) (end 91.2 85) (width 0.15) (layer B.Cu) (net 5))
 (segment (start 89.15 83.05) (end 88.8 82.7) (width 0.15) (layer B.Cu) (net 10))
 (segment (start 89.15 84.5) (end 89.15 83.05) (width 0.15) (layer B.Cu) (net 10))
 (via (at 89.7 83.4) (size 0.45) (drill 0.2) (layers F.Cu B.Cu) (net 10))
 (segment (start 89 82.7) (end 89.7 83.4) (width 0.15) (layer B.Cu) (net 10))
 (segment (start 88.8 82.7) (end 89 82.7) (width 0.15) (layer B.Cu) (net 10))
 (segment (start 90.825 83.4) (end 91 83.225) (width 0.15) (layer F.Cu) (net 10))
 (segment (start 89.7 83.4) (end 90.825 83.4) (width 0.15) (layer F.Cu) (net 10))
 (segment (start 92.35 81) (end 92.35 83) (width 0.15) (layer B.Cu) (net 3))
 (segment (start 92.2 83.15) (end 92.2 82.95) (width 0.2) (layer B.Cu) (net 3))
 (segment (start 93.55 84.5) (end 92.2 83.15) (width 0.2) (layer B.Cu) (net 3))
 (segment (start 95.5 84.5) (end 93.55 84.5) (width 0.2) (layer B.Cu) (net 3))
 (segment (start 92.35 82.8) (end 92.2 82.95) (width 0.2) (layer B.Cu) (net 3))
 (segment (start 92.35 81) (end 92.35 82.8) (width 0.2) (layer B.Cu) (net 3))
 (segment (start 91.175 82.95) (end 90.925 82.7) (width 0.2) (layer B.Cu) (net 3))
 (segment (start 92.2 82.95) (end 91.175 82.95) (width 0.2) (layer B.Cu) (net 3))
 (segment (start 89.3 81) (end 90.7 81) (width 0.15) (layer B.Cu) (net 1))
 (segment (start 90.7 81) (end 90.7 81.09721) (width 0.15) (layer B.Cu) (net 1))
 (via (at 89.690398 82.106812) (size 0.45) (drill 0.2) (layers F.Cu B.Cu) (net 1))
 (segment (start 90.7 81.09721) (end 89.690398 82.106812) (width 0.15) (layer B.Cu) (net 1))
 (segment (start 89.690398 82.290398) (end 89.690398 82.106812) (width 0.15) (layer F.Cu) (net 1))
 (segment (start 91 82.575) (end 89.975 82.575) (width 0.15) (layer F.Cu) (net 1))
 (segment (start 89.975 82.575) (end 89.690398 82.290398) (width 0.15) (layer F.Cu) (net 1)))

